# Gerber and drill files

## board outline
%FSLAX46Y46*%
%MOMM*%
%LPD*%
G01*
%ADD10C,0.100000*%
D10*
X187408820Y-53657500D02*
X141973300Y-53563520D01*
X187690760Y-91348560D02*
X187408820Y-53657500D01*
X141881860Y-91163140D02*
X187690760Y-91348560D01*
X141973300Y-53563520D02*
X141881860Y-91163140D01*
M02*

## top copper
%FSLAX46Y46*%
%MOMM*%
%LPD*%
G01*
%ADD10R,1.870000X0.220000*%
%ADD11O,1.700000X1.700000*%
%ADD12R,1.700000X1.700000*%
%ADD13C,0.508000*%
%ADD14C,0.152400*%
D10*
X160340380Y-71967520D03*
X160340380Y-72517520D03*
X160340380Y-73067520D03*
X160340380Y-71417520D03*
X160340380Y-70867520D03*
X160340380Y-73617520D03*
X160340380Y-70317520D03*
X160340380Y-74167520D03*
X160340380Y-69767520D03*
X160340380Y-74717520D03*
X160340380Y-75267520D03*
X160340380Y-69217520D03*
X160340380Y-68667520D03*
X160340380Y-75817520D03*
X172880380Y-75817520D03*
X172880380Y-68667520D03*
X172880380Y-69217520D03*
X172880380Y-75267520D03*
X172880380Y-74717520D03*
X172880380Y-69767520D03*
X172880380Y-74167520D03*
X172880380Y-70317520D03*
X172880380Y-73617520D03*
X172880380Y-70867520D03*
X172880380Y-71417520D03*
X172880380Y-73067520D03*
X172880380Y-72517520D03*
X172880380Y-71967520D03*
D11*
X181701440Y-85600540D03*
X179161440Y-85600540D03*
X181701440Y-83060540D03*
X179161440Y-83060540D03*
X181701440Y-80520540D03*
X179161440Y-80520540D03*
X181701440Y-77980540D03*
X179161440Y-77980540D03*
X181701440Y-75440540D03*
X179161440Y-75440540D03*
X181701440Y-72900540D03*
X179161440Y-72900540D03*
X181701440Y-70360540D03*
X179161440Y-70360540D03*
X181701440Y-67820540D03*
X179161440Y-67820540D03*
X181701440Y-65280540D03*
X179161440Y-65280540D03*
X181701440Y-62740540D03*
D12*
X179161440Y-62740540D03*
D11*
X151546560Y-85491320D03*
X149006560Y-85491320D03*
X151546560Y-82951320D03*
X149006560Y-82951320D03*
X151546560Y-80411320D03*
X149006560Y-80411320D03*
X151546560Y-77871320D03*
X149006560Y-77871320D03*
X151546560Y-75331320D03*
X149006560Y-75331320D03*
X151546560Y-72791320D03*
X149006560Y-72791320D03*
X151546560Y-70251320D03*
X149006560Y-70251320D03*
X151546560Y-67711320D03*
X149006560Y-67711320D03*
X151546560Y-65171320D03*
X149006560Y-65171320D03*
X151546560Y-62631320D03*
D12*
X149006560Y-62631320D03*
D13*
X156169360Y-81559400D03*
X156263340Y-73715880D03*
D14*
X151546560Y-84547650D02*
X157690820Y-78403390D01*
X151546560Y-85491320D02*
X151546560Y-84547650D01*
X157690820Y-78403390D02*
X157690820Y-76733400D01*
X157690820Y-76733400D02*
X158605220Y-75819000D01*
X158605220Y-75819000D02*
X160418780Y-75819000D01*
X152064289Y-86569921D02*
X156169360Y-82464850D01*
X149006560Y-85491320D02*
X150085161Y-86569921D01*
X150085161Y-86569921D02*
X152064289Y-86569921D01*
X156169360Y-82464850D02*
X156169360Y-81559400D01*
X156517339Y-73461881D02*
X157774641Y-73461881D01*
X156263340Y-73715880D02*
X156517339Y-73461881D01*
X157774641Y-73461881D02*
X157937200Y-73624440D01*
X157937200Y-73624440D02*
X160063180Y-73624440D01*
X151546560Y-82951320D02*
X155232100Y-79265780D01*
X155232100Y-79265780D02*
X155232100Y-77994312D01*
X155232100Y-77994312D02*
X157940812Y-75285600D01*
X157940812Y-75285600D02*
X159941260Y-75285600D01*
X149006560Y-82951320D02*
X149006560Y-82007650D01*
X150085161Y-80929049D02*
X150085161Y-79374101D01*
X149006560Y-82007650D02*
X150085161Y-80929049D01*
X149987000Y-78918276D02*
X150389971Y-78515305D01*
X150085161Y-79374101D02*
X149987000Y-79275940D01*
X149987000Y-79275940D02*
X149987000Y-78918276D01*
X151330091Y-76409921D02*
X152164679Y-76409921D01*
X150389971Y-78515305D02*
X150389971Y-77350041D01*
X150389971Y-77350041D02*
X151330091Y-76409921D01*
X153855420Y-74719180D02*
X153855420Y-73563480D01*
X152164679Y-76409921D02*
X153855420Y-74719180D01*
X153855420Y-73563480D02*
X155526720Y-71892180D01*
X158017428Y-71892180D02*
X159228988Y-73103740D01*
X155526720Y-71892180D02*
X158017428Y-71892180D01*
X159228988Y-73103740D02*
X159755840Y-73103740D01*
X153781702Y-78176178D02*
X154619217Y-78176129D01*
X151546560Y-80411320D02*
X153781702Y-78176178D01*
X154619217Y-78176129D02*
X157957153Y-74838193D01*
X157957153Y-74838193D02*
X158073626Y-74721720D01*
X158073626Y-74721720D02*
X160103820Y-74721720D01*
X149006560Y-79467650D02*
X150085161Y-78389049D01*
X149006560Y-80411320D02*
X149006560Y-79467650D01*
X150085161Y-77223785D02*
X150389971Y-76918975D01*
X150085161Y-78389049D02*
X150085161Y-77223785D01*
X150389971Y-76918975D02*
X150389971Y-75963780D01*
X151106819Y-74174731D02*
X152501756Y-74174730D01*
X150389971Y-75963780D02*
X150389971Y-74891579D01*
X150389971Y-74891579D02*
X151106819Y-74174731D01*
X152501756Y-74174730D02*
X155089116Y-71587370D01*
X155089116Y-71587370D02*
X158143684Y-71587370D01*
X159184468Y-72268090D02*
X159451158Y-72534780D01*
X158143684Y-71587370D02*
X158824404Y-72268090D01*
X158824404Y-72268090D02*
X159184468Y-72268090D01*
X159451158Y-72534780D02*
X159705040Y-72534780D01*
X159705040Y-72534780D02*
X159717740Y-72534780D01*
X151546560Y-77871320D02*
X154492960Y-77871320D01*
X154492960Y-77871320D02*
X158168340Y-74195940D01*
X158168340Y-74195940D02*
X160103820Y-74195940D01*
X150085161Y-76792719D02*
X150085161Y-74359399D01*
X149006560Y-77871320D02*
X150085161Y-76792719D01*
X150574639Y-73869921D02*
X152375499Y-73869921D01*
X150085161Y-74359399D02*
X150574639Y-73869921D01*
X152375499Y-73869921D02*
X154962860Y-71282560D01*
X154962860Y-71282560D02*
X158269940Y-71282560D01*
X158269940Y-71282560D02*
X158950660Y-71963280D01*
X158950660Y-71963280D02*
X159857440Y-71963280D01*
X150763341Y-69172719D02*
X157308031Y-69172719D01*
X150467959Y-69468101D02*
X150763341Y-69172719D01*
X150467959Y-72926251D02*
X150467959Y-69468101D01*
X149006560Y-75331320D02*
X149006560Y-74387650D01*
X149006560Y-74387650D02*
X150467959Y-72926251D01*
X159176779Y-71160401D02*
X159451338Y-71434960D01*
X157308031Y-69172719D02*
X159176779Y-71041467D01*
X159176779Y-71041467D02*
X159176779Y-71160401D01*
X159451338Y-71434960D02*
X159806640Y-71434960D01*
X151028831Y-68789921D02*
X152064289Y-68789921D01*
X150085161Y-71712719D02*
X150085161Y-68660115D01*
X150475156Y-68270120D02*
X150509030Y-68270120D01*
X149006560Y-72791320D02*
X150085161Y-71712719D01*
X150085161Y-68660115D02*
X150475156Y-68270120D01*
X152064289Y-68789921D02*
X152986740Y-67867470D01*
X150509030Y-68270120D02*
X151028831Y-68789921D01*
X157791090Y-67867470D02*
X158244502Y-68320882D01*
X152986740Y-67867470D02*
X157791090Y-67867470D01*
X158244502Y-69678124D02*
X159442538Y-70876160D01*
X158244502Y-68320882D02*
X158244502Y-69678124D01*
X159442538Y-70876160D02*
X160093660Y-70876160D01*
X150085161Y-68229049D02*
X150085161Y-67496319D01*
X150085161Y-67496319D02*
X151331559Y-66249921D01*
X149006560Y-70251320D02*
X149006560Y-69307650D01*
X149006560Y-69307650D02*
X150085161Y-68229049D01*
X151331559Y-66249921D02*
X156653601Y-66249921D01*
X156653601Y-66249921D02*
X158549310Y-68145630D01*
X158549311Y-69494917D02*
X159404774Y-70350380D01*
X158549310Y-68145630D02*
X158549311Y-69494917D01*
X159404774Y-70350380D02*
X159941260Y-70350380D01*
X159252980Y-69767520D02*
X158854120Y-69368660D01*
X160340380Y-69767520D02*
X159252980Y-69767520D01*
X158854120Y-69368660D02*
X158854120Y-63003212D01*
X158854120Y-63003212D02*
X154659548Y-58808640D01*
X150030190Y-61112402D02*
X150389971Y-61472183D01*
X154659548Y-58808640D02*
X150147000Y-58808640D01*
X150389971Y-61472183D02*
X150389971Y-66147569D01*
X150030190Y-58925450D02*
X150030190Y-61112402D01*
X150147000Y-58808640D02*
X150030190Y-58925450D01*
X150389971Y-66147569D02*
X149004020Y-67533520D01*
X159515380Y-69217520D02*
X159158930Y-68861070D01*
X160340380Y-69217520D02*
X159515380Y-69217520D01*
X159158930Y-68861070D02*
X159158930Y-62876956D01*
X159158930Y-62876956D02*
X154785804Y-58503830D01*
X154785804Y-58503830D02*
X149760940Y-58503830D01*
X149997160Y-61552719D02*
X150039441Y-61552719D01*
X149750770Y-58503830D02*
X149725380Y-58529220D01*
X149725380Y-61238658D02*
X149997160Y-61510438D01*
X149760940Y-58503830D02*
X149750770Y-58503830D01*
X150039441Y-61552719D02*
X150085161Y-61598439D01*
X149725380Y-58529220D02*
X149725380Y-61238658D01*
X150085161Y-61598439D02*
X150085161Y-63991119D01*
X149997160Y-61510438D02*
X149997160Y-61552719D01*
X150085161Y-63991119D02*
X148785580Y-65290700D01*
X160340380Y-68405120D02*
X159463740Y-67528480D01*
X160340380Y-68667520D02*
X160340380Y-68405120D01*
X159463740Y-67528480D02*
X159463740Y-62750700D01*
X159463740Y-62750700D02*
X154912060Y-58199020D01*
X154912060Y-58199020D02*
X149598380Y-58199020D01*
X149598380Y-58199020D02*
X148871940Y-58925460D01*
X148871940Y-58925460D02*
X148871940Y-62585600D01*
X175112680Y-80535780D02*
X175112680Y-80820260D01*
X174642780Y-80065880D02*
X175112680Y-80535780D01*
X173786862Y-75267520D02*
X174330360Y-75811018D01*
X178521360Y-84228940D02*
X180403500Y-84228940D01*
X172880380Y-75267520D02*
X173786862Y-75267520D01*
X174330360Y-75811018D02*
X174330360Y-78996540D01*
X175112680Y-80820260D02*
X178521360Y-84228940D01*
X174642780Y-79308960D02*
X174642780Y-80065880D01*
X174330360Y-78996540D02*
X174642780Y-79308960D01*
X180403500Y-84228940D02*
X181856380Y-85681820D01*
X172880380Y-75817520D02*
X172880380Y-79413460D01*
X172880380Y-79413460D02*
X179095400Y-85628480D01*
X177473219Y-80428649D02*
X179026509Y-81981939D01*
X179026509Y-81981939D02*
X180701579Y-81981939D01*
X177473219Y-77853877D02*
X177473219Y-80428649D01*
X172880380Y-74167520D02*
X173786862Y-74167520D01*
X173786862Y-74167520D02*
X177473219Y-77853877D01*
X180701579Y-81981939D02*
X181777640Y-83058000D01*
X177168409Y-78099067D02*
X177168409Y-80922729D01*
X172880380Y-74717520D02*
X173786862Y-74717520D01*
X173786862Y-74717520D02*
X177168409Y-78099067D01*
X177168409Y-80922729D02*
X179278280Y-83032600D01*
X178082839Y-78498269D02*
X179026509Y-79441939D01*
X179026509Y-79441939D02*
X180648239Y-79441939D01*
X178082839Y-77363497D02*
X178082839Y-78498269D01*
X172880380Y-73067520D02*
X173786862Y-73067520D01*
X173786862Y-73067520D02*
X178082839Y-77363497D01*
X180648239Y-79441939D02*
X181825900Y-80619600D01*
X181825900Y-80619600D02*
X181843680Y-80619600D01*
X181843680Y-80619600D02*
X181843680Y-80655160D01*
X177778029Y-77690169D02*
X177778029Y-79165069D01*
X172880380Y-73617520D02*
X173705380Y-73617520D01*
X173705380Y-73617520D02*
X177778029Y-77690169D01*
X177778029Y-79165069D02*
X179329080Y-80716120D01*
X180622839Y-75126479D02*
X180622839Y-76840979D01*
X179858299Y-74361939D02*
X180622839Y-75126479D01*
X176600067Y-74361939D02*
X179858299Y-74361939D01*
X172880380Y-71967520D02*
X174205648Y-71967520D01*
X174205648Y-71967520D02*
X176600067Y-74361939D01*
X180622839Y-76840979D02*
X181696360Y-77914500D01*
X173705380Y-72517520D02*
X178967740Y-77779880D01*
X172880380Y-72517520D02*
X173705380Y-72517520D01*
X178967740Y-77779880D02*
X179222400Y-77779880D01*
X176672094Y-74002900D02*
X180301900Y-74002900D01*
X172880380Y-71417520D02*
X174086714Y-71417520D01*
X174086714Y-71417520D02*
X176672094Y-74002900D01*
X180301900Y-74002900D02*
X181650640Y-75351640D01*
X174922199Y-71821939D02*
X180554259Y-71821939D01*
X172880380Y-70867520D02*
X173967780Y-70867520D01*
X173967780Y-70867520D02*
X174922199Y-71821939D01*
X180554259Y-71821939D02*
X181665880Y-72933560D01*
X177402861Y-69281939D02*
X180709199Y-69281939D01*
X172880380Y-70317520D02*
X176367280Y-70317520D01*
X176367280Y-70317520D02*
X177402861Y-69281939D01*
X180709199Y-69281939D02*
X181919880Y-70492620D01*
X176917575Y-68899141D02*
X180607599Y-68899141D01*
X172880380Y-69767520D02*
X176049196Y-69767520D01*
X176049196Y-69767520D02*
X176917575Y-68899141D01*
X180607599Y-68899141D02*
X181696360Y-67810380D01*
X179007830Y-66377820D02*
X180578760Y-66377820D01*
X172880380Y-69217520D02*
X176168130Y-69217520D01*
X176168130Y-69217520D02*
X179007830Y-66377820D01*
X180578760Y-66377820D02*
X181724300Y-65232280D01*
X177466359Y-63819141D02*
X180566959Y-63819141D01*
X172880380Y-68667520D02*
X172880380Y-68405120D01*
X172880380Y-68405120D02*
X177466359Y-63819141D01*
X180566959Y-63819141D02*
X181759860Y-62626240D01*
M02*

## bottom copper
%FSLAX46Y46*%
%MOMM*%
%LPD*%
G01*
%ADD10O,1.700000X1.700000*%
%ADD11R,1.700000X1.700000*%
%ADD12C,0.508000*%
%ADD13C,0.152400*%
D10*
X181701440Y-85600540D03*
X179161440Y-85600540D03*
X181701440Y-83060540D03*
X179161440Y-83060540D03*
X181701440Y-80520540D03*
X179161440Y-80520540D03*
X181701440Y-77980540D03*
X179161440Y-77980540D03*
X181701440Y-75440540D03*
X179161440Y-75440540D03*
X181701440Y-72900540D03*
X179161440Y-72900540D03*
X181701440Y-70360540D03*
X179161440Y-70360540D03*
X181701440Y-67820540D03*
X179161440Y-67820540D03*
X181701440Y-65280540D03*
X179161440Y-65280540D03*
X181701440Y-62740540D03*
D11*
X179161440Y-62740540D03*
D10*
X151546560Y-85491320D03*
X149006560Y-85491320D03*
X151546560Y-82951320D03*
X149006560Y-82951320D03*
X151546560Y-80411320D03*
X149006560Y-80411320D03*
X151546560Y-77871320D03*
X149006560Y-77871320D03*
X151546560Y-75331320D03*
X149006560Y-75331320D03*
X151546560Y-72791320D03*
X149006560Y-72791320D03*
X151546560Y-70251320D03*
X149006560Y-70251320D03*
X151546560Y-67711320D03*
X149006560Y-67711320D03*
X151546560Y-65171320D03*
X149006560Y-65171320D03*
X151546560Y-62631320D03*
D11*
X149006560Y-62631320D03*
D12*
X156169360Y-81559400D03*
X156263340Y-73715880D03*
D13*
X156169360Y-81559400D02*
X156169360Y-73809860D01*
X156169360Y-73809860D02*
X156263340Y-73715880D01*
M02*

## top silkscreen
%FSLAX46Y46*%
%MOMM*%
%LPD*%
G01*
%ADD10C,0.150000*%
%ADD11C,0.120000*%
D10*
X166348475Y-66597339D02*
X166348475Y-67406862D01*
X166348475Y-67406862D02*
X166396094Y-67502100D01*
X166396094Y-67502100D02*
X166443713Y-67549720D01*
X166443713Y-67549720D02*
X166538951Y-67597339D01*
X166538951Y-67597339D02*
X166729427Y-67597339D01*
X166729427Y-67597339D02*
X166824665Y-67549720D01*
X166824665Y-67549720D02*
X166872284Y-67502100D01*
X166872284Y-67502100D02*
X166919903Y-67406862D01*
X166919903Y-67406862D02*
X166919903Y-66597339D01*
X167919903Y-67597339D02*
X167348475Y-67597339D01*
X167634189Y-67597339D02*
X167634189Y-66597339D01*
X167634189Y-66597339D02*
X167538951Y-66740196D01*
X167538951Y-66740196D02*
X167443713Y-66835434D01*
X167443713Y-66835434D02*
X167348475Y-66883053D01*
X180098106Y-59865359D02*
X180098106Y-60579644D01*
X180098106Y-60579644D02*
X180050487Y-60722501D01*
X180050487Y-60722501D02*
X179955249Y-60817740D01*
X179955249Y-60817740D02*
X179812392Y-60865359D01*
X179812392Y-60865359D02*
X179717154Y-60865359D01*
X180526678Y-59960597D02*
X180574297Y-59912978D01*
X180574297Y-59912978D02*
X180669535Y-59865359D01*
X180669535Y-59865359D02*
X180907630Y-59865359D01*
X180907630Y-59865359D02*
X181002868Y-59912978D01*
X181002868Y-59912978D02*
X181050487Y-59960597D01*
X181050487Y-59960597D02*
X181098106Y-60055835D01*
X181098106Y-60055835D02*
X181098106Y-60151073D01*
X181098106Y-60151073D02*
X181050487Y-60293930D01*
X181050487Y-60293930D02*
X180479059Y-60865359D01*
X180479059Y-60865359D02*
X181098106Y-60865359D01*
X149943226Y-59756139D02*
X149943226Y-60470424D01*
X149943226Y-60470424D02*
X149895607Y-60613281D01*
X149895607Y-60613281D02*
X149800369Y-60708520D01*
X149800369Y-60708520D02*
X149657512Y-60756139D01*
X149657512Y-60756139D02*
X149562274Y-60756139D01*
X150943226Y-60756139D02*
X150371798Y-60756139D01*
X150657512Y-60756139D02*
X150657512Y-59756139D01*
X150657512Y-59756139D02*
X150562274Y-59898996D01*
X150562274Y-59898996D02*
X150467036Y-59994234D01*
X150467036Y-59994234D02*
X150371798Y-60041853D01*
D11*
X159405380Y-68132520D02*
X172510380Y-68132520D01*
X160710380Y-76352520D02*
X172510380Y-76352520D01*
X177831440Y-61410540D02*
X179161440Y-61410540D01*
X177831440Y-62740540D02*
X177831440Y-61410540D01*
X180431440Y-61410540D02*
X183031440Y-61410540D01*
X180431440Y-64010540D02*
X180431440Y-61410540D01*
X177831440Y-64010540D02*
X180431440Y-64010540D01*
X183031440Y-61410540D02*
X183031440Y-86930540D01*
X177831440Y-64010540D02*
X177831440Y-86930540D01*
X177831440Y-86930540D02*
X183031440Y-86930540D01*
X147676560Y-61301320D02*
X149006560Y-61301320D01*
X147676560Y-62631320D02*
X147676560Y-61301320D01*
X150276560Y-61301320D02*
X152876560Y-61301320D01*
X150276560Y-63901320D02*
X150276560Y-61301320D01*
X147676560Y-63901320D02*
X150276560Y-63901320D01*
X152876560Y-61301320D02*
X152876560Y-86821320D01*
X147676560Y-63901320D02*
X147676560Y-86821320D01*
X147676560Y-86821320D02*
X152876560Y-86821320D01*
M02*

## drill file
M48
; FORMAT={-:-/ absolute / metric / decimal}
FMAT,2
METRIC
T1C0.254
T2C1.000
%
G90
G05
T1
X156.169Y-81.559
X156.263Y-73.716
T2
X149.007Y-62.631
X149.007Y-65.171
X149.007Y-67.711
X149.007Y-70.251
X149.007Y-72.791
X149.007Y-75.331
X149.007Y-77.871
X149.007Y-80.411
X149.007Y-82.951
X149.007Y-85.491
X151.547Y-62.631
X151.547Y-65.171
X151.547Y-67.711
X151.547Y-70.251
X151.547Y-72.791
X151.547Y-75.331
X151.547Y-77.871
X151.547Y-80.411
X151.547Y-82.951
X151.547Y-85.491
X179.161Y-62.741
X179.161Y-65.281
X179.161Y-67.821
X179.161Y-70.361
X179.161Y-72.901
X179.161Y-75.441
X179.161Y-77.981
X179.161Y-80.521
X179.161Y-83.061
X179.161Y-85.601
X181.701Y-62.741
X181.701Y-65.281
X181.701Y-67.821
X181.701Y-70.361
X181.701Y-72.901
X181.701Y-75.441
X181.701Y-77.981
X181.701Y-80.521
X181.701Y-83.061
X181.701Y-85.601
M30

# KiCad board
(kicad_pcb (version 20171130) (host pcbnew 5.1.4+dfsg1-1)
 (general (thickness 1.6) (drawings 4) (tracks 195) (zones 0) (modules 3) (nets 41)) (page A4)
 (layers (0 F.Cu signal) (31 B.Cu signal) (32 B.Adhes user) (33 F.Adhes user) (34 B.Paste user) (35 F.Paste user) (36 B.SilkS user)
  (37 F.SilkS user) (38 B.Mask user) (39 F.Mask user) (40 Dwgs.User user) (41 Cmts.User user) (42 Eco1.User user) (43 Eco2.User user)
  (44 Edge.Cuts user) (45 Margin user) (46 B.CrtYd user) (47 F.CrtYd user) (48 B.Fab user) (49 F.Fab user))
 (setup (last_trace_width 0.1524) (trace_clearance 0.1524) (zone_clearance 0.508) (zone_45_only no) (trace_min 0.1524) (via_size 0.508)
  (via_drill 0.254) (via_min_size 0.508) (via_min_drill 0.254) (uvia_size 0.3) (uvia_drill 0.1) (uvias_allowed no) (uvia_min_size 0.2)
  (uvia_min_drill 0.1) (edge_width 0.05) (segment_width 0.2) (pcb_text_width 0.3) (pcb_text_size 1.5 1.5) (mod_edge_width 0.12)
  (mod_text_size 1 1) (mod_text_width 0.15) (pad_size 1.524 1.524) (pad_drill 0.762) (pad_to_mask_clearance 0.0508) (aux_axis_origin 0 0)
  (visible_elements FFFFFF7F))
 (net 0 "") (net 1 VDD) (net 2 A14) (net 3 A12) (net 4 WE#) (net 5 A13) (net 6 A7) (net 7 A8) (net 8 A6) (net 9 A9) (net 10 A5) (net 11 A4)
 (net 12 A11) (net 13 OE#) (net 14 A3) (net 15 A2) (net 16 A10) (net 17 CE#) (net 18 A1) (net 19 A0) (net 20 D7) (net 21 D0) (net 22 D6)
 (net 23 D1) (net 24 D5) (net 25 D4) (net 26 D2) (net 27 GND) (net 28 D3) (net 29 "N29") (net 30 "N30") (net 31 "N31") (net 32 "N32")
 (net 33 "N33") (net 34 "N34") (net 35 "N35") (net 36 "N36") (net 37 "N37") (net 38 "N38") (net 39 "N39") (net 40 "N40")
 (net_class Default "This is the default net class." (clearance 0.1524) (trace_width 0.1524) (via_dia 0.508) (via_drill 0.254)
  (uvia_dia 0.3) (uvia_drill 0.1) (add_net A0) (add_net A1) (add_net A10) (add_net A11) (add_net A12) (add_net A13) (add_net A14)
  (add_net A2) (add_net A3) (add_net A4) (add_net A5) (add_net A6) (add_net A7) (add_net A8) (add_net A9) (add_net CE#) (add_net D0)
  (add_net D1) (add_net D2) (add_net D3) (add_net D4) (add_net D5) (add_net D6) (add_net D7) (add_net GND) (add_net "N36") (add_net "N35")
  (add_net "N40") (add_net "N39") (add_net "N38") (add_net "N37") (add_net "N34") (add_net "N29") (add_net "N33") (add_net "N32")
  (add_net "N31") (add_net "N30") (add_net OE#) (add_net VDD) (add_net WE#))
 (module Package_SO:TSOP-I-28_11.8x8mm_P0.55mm (layer F.Cu) (at 166.61038 72.24252)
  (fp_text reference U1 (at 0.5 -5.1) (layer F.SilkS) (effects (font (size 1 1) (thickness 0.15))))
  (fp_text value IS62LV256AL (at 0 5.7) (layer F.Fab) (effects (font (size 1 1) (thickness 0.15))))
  (fp_line (start -7.205 -4.11) (end 5.9 -4.11) (layer F.SilkS) (width 0.12))
  (fp_line (start -5.9 4.11) (end 5.9 4.11) (layer F.SilkS) (width 0.12))
  (pad 7 smd rect (at -6.27 -0.275) (size 1.87 0.22) (layers F.Cu F.Paste F.Mask) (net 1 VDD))
  (pad 8 smd rect (at -6.27 0.275) (size 1.87 0.22) (layers F.Cu F.Paste F.Mask) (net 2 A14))
  (pad 9 smd rect (at -6.27 0.825) (size 1.87 0.22) (layers F.Cu F.Paste F.Mask) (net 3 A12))
  (pad 6 smd rect (at -6.27 -0.825) (size 1.87 0.22) (layers F.Cu F.Paste F.Mask) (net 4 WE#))
  (pad 5 smd rect (at -6.27 -1.375) (size 1.87 0.22) (layers F.Cu F.Paste F.Mask) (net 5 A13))
  (pad 10 smd rect (at -6.27 1.375) (size 1.87 0.22) (layers F.Cu F.Paste F.Mask) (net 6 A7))
  (pad 4 smd rect (at -6.27 -1.925) (size 1.87 0.22) (layers F.Cu F.Paste F.Mask) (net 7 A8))
  (pad 11 smd rect (at -6.27 1.925) (size 1.87 0.22) (layers F.Cu F.Paste F.Mask) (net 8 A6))
  (pad 3 smd rect (at -6.27 -2.475) (size 1.87 0.22) (layers F.Cu F.Paste F.Mask) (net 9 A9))
  (pad 12 smd rect (at -6.27 2.475) (size 1.87 0.22) (layers F.Cu F.Paste F.Mask) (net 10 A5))
  (pad 13 smd rect (at -6.27 3.025) (size 1.87 0.22) (layers F.Cu F.Paste F.Mask) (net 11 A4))
  (pad 2 smd rect (at -6.27 -3.025) (size 1.87 0.22) (layers F.Cu F.Paste F.Mask) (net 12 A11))
  (pad 1 smd rect (at -6.27 -3.575) (size 1.87 0.22) (layers F.Cu F.Paste F.Mask) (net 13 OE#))
  (pad 14 smd rect (at -6.27 3.575) (size 1.87 0.22) (layers F.Cu F.Paste F.Mask) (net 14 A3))
  (pad 15 smd rect (at 6.27 3.575) (size 1.87 0.22) (layers F.Cu F.Paste F.Mask) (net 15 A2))
  (pad 28 smd rect (at 6.27 -3.575) (size 1.87 0.22) (layers F.Cu F.Paste F.Mask) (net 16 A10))
  (pad 27 smd rect (at 6.27 -3.025) (size 1.87 0.22) (layers F.Cu F.Paste F.Mask) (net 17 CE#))
  (pad 16 smd rect (at 6.27 3.025) (size 1.87 0.22) (layers F.Cu F.Paste F.Mask) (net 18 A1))
  (pad 17 smd rect (at 6.27 2.475) (size 1.87 0.22) (layers F.Cu F.Paste F.Mask) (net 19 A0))
  (pad 26 smd rect (at 6.27 -2.475) (size 1.87 0.22) (layers F.Cu F.Paste F.Mask) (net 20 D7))
  (pad 18 smd rect (at 6.27 1.925) (size 1.87 0.22) (layers F.Cu F.Paste F.Mask) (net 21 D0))
  (pad 25 smd rect (at 6.27 -1.925) (size 1.87 0.22) (layers F.Cu F.Paste F.Mask) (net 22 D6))
  (pad 19 smd rect (at 6.27 1.375) (size 1.87 0.22) (layers F.Cu F.Paste F.Mask) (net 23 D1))
  (pad 24 smd rect (at 6.27 -1.375) (size 1.87 0.22) (layers F.Cu F.Paste F.Mask) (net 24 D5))
  (pad 23 smd rect (at 6.27 -0.825) (size 1.87 0.22) (layers F.Cu F.Paste F.Mask) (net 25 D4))
  (pad 20 smd rect (at 6.27 0.825) (size 1.87 0.22) (layers F.Cu F.Paste F.Mask) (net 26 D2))
  (pad 21 smd rect (at 6.27 0.275) (size 1.87 0.22) (layers F.Cu F.Paste F.Mask) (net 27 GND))
  (pad 22 smd rect (at 6.27 -0.275) (size 1.87 0.22) (layers F.Cu F.Paste F.Mask) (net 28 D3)))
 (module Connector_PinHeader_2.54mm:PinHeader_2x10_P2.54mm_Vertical (layer F.Cu) (at 179.16144 62.74054)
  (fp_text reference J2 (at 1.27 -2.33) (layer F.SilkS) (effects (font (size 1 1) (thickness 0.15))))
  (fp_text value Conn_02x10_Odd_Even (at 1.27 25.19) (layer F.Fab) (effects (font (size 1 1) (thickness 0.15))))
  (fp_line (start -1.33 -1.33) (end 0 -1.33) (layer F.SilkS) (width 0.12))
  (fp_line (start -1.33 0) (end -1.33 -1.33) (layer F.SilkS) (width 0.12))
  (fp_line (start 1.27 -1.33) (end 3.87 -1.33) (layer F.SilkS) (width 0.12))
  (fp_line (start 1.27 1.27) (end 1.27 -1.33) (layer F.SilkS) (width 0.12))
  (fp_line (start -1.33 1.27) (end 1.27 1.27) (layer F.SilkS) (width 0.12))
  (fp_line (start 3.87 -1.33) (end 3.87 24.19) (layer F.SilkS) (width 0.12))
  (fp_line (start -1.33 1.27) (end -1.33 24.19) (layer F.SilkS) (width 0.12))
  (fp_line (start -1.33 24.19) (end 3.87 24.19) (layer F.SilkS) (width 0.12))
  (pad 20 thru_hole oval (at 2.54 22.86) (size 1.7 1.7) (drill 1) (layers *.Cu *.Mask) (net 18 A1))
  (pad 19 thru_hole oval (at 0 22.86) (size 1.7 1.7) (drill 1) (layers *.Cu *.Mask) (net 15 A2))
  (pad 18 thru_hole oval (at 2.54 20.32) (size 1.7 1.7) (drill 1) (layers *.Cu *.Mask) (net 21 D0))
  (pad 17 thru_hole oval (at 0 20.32) (size 1.7 1.7) (drill 1) (layers *.Cu *.Mask) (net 19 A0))
  (pad 16 thru_hole oval (at 2.54 17.78) (size 1.7 1.7) (drill 1) (layers *.Cu *.Mask) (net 26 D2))
  (pad 15 thru_hole oval (at 0 17.78) (size 1.7 1.7) (drill 1) (layers *.Cu *.Mask) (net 23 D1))
  (pad 14 thru_hole oval (at 2.54 15.24) (size 1.7 1.7) (drill 1) (layers *.Cu *.Mask) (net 28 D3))
  (pad 13 thru_hole oval (at 0 15.24) (size 1.7 1.7) (drill 1) (layers *.Cu *.Mask) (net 27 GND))
  (pad 12 thru_hole oval (at 2.54 12.7) (size 1.7 1.7) (drill 1) (layers *.Cu *.Mask) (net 25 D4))
  (pad 11 thru_hole oval (at 0 12.7) (size 1.7 1.7) (drill 1) (layers *.Cu *.Mask) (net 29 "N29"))
  (pad 10 thru_hole oval (at 2.54 10.16) (size 1.7 1.7) (drill 1) (layers *.Cu *.Mask) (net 24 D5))
  (pad 9 thru_hole oval (at 0 10.16) (size 1.7 1.7) (drill 1) (layers *.Cu *.Mask) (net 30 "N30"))
  (pad 8 thru_hole oval (at 2.54 7.62) (size 1.7 1.7) (drill 1) (layers *.Cu *.Mask) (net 22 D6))
  (pad 7 thru_hole oval (at 0 7.62) (size 1.7 1.7) (drill 1) (layers *.Cu *.Mask) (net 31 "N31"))
  (pad 6 thru_hole oval (at 2.54 5.08) (size 1.7 1.7) (drill 1) (layers *.Cu *.Mask) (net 20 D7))
  (pad 5 thru_hole oval (at 0 5.08) (size 1.7 1.7) (drill 1) (layers *.Cu *.Mask) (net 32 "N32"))
  (pad 4 thru_hole oval (at 2.54 2.54) (size 1.7 1.7) (drill 1) (layers *.Cu *.Mask) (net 17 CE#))
  (pad 3 thru_hole oval (at 0 2.54) (size 1.7 1.7) (drill 1) (layers *.Cu *.Mask) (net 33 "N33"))
  (pad 2 thru_hole oval (at 2.54 0) (size 1.7 1.7) (drill 1) (layers *.Cu *.Mask) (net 16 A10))
  (pad 1 thru_hole rect (at 0 0) (size 1.7 1.7) (drill 1) (layers *.Cu *.Mask) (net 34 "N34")))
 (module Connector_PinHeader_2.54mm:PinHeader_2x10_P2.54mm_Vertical (layer F.Cu) (at 149.00656 62.63132)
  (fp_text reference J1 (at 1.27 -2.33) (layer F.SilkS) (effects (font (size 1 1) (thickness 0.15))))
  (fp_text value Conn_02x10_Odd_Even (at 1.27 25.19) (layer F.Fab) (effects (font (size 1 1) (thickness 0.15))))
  (fp_line (start -1.33 -1.33) (end 0 -1.33) (layer F.SilkS) (width 0.12))
  (fp_line (start -1.33 0) (end -1.33 -1.33) (layer F.SilkS) (width 0.12))
  (fp_line (start 1.27 -1.33) (end 3.87 -1.33) (layer F.SilkS) (width 0.12))
  (fp_line (start 1.27 1.27) (end 1.27 -1.33) (layer F.SilkS) (width 0.12))
  (fp_line (start -1.33 1.27) (end 1.27 1.27) (layer F.SilkS) (width 0.12))
  (fp_line (start 3.87 -1.33) (end 3.87 24.19) (layer F.SilkS) (width 0.12))
  (fp_line (start -1.33 1.27) (end -1.33 24.19) (layer F.SilkS) (width 0.12))
  (fp_line (start -1.33 24.19) (end 3.87 24.19) (layer F.SilkS) (width 0.12))
  (pad 20 thru_hole oval (at 2.54 22.86) (size 1.7 1.7) (drill 1) (layers *.Cu *.Mask) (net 14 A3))
  (pad 19 thru_hole oval (at 0 22.86) (size 1.7 1.7) (drill 1) (layers *.Cu *.Mask) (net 6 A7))
  (pad 18 thru_hole oval (at 2.54 20.32) (size 1.7 1.7) (drill 1) (layers *.Cu *.Mask) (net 11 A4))
  (pad 17 thru_hole oval (at 0 20.32) (size 1.7 1.7) (drill 1) (layers *.Cu *.Mask) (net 3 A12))
  (pad 16 thru_hole oval (at 2.54 17.78) (size 1.7 1.7) (drill 1) (layers *.Cu *.Mask) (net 10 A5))
  (pad 15 thru_hole oval (at 0 17.78) (size 1.7 1.7) (drill 1) (layers *.Cu *.Mask) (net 2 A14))
  (pad 14 thru_hole oval (at 2.54 15.24) (size 1.7 1.7) (drill 1) (layers *.Cu *.Mask) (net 8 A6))
  (pad 13 thru_hole oval (at 0 15.24) (size 1.7 1.7) (drill 1) (layers *.Cu *.Mask) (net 1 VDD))
  (pad 12 thru_hole oval (at 2.54 12.7) (size 1.7 1.7) (drill 1) (layers *.Cu *.Mask) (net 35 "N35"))
  (pad 11 thru_hole oval (at 0 12.7) (size 1.7 1.7) (drill 1) (layers *.Cu *.Mask) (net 4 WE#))
  (pad 10 thru_hole oval (at 2.54 10.16) (size 1.7 1.7) (drill 1) (layers *.Cu *.Mask) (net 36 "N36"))
  (pad 9 thru_hole oval (at 0 10.16) (size 1.7 1.7) (drill 1) (layers *.Cu *.Mask) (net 5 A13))
  (pad 8 thru_hole oval (at 2.54 7.62) (size 1.7 1.7) (drill 1) (layers *.Cu *.Mask) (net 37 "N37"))
  (pad 7 thru_hole oval (at 0 7.62) (size 1.7 1.7) (drill 1) (layers *.Cu *.Mask) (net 7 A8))
  (pad 6 thru_hole oval (at 2.54 5.08) (size 1.7 1.7) (drill 1) (layers *.Cu *.Mask) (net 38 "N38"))
  (pad 5 thru_hole oval (at 0 5.08) (size 1.7 1.7) (drill 1) (layers *.Cu *.Mask) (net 9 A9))
  (pad 4 thru_hole oval (at 2.54 2.54) (size 1.7 1.7) (drill 1) (layers *.Cu *.Mask) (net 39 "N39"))
  (pad 3 thru_hole oval (at 0 2.54) (size 1.7 1.7) (drill 1) (layers *.Cu *.Mask) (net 12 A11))
  (pad 2 thru_hole oval (at 2.54 0) (size 1.7 1.7) (drill 1) (layers *.Cu *.Mask) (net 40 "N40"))
  (pad 1 thru_hole rect (at 0 0) (size 1.7 1.7) (drill 1) (layers *.Cu *.Mask) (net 13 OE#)))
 (gr_line (start 187.40882 53.6575) (end 141.9733 53.56352) (layer Edge.Cuts) (width 0.1))
 (gr_line (start 187.69076 91.34856) (end 187.40882 53.6575) (layer Edge.Cuts) (width 0.1))
 (gr_line (start 141.88186 91.16314) (end 187.69076 91.34856) (layer Edge.Cuts) (width 0.1))
 (gr_line (start 141.9733 53.56352) (end 141.88186 91.16314) (layer Edge.Cuts) (width 0.1))
 (segment (start 151.54656 84.54765) (end 157.69082 78.40339) (width 0.1524) (layer F.Cu) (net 14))
 (segment (start 151.54656 85.49132) (end 151.54656 84.54765) (width 0.1524) (layer F.Cu) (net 14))
 (segment (start 157.69082 78.40339) (end 157.69082 76.7334) (width 0.1524) (layer F.Cu) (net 14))
 (segment (start 157.69082 76.7334) (end 158.60522 75.819) (width 0.1524) (layer F.Cu) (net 14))
 (segment (start 158.60522 75.819) (end 160.41878 75.819) (width 0.1524) (layer F.Cu) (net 14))
 (segment (start 152.064289 86.569921) (end 156.16936 82.46485) (width 0.1524) (layer F.Cu) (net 6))
 (segment (start 149.00656 85.49132) (end 150.085161 86.569921) (width 0.1524) (layer F.Cu) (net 6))
 (segment (start 150.085161 86.569921) (end 152.064289 86.569921) (width 0.1524) (layer F.Cu) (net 6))
 (via (at 156.16936 81.5594) (size 0.508) (drill 0.254) (layers F.Cu B.Cu) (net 6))
 (segment (start 156.16936 82.46485) (end 156.16936 81.5594) (width 0.1524) (layer F.Cu) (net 6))
 (via (at 156.26334 73.71588) (size 0.508) (drill 0.254) (layers F.Cu B.Cu) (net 6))
 (segment (start 156.16936 81.5594) (end 156.16936 73.80986) (width 0.1524) (layer B.Cu) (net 6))
 (segment (start 156.16936 73.80986) (end 156.26334 73.71588) (width 0.1524) (layer B.Cu) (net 6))
 (segment (start 156.517339 73.461881) (end 157.774641 73.461881) (width 0.1524) (layer F.Cu) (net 6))
 (segment (start 156.26334 73.71588) (end 156.517339 73.461881) (width 0.1524) (layer F.Cu) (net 6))
 (segment (start 157.774641 73.461881) (end 157.9372 73.62444) (width 0.1524) (layer F.Cu) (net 6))
 (segment (start 157.9372 73.62444) (end 160.06318 73.62444) (width 0.1524) (layer F.Cu) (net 6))
 (segment (start 151.54656 82.95132) (end 155.2321 79.26578) (width 0.1524) (layer F.Cu) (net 11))
 (segment (start 155.2321 79.26578) (end 155.2321 77.994312) (width 0.1524) (layer F.Cu) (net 11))
 (segment (start 155.2321 77.994312) (end 157.940812 75.2856) (width 0.1524) (layer F.Cu) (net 11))
 (segment (start 157.940812 75.2856) (end 159.94126 75.2856) (width 0.1524) (layer F.Cu) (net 11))
 (segment (start 149.00656 82.95132) (end 149.00656 82.00765) (width 0.1524) (layer F.Cu) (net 3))
 (segment (start 150.085161 80.929049) (end 150.085161 79.374101) (width 0.1524) (layer F.Cu) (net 3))
 (segment (start 149.00656 82.00765) (end 150.085161 80.929049) (width 0.1524) (layer F.Cu) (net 3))
 (segment (start 149.987 78.918276) (end 150.389971 78.515305) (width 0.1524) (layer F.Cu) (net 3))
 (segment (start 150.085161 79.374101) (end 149.987 79.27594) (width 0.1524) (layer F.Cu) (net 3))
 (segment (start 149.987 79.27594) (end 149.987 78.918276) (width 0.1524) (layer F.Cu) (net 3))
 (segment (start 151.330091 76.409921) (end 152.164679 76.409921) (width 0.1524) (layer F.Cu) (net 3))
 (segment (start 150.389971 78.515305) (end 150.389971 77.350041) (width 0.1524) (layer F.Cu) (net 3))
 (segment (start 150.389971 77.350041) (end 151.330091 76.409921) (width 0.1524) (layer F.Cu) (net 3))
 (segment (start 153.85542 74.71918) (end 153.85542 73.56348) (width 0.1524) (layer F.Cu) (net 3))
 (segment (start 152.164679 76.409921) (end 153.85542 74.71918) (width 0.1524) (layer F.Cu) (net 3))
 (segment (start 153.85542 73.56348) (end 155.52672 71.89218) (width 0.1524) (layer F.Cu) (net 3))
 (segment (start 158.017428 71.89218) (end 159.228988 73.10374) (width 0.1524) (layer F.Cu) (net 3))
 (segment (start 155.52672 71.89218) (end 158.017428 71.89218) (width 0.1524) (layer F.Cu) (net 3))
 (segment (start 159.228988 73.10374) (end 159.75584 73.10374) (width 0.1524) (layer F.Cu) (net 3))
 (segment (start 153.781702 78.176178) (end 154.619217 78.176129) (width 0.1524) (layer F.Cu) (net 10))
 (segment (start 151.54656 80.41132) (end 153.781702 78.176178) (width 0.1524) (layer F.Cu) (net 10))
 (segment (start 154.619217 78.176129) (end 157.957153 74.838193) (width 0.1524) (layer F.Cu) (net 10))
 (segment (start 157.957153 74.838193) (end 158.073626 74.72172) (width 0.1524) (layer F.Cu) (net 10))
 (segment (start 158.073626 74.72172) (end 160.10382 74.72172) (width 0.1524) (layer F.Cu) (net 10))
 (segment (start 149.00656 79.46765) (end 150.085161 78.389049) (width 0.1524) (layer F.Cu) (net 2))
 (segment (start 149.00656 80.41132) (end 149.00656 79.46765) (width 0.1524) (layer F.Cu) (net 2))
 (segment (start 150.085161 77.223785) (end 150.389971 76.918975) (width 0.1524) (layer F.Cu) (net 2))
 (segment (start 150.085161 78.389049) (end 150.085161 77.223785) (width 0.1524) (layer F.Cu) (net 2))
 (segment (start 150.389971 76.918975) (end 150.389971 75.96378) (width 0.1524) (layer F.Cu) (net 2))
 (segment (start 151.106819 74.174731) (end 152.501756 74.17473) (width 0.1524) (layer F.Cu) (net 2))
 (segment (start 150.389971 75.96378) (end 150.389971 74.891579) (width 0.1524) (layer F.Cu) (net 2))
 (segment (start 150.389971 74.891579) (end 151.106819 74.174731) (width 0.1524) (layer F.Cu) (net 2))
 (segment (start 152.501756 74.17473) (end 155.089116 71.58737) (width 0.1524) (layer F.Cu) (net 2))
 (segment (start 155.089116 71.58737) (end 158.143684 71.58737) (width 0.1524) (layer F.Cu) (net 2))
 (segment (start 159.184468 72.26809) (end 159.451158 72.53478) (width 0.1524) (layer F.Cu) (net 2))
 (segment (start 158.143684 71.58737) (end 158.824404 72.26809) (width 0.1524) (layer F.Cu) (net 2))
 (segment (start 158.824404 72.26809) (end 159.184468 72.26809) (width 0.1524) (layer F.Cu) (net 2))
 (segment (start 159.451158 72.53478) (end 159.70504 72.53478) (width 0.1524) (layer F.Cu) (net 2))
 (segment (start 159.70504 72.53478) (end 159.71774 72.53478) (width 0.1524) (layer F.Cu) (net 2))
 (segment (start 151.54656 77.87132) (end 154.49296 77.87132) (width 0.1524) (layer F.Cu) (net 8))
 (segment (start 154.49296 77.87132) (end 158.16834 74.19594) (width 0.1524) (layer F.Cu) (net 8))
 (segment (start 158.16834 74.19594) (end 160.10382 74.19594) (width 0.1524) (layer F.Cu) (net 8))
 (segment (start 150.085161 76.792719) (end 150.085161 74.359399) (width 0.1524) (layer F.Cu) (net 1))
 (segment (start 149.00656 77.87132) (end 150.085161 76.792719) (width 0.1524) (layer F.Cu) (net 1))
 (segment (start 150.574639 73.869921) (end 152.375499 73.869921) (width 0.1524) (layer F.Cu) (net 1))
 (segment (start 150.085161 74.359399) (end 150.574639 73.869921) (width 0.1524) (layer F.Cu) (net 1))
 (segment (start 152.375499 73.869921) (end 154.96286 71.28256) (width 0.1524) (layer F.Cu) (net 1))
 (segment (start 154.96286 71.28256) (end 158.26994 71.28256) (width 0.1524) (layer F.Cu) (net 1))
 (segment (start 158.26994 71.28256) (end 158.95066 71.96328) (width 0.1524) (layer F.Cu) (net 1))
 (segment (start 158.95066 71.96328) (end 159.85744 71.96328) (width 0.1524) (layer F.Cu) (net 1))
 (segment (start 150.763341 69.172719) (end 157.308031 69.172719) (width 0.1524) (layer F.Cu) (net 4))
 (segment (start 150.467959 69.468101) (end 150.763341 69.172719) (width 0.1524) (layer F.Cu) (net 4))
 (segment (start 150.467959 72.926251) (end 150.467959 69.468101) (width 0.1524) (layer F.Cu) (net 4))
 (segment (start 149.00656 75.33132) (end 149.00656 74.38765) (width 0.1524) (layer F.Cu) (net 4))
 (segment (start 149.00656 74.38765) (end 150.467959 72.926251) (width 0.1524) (layer F.Cu) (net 4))
 (segment (start 159.176779 71.160401) (end 159.451338 71.43496) (width 0.1524) (layer F.Cu) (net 4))
 (segment (start 157.308031 69.172719) (end 159.176779 71.041467) (width 0.1524) (layer F.Cu) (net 4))
 (segment (start 159.176779 71.041467) (end 159.176779 71.160401) (width 0.1524) (layer F.Cu) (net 4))
 (segment (start 159.451338 71.43496) (end 159.80664 71.43496) (width 0.1524) (layer F.Cu) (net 4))
 (segment (start 151.028831 68.789921) (end 152.064289 68.789921) (width 0.1524) (layer F.Cu) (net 5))
 (segment (start 150.085161 71.712719) (end 150.085161 68.660115) (width 0.1524) (layer F.Cu) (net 5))
 (segment (start 150.475156 68.27012) (end 150.50903 68.27012) (width 0.1524) (layer F.Cu) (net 5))
 (segment (start 149.00656 72.79132) (end 150.085161 71.712719) (width 0.1524) (layer F.Cu) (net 5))
 (segment (start 150.085161 68.660115) (end 150.475156 68.27012) (width 0.1524) (layer F.Cu) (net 5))
 (segment (start 152.064289 68.789921) (end 152.98674 67.86747) (width 0.1524) (layer F.Cu) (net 5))
 (segment (start 150.50903 68.27012) (end 151.028831 68.789921) (width 0.1524) (layer F.Cu) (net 5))
 (segment (start 157.79109 67.86747) (end 158.244502 68.320882) (width 0.1524) (layer F.Cu) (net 5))
 (segment (start 152.98674 67.86747) (end 157.79109 67.86747) (width 0.1524) (layer F.Cu) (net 5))
 (segment (start 158.244502 69.678124) (end 159.442538 70.87616) (width 0.1524) (layer F.Cu) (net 5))
 (segment (start 158.244502 68.320882) (end 158.244502 69.678124) (width 0.1524) (layer F.Cu) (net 5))
 (segment (start 159.442538 70.87616) (end 160.09366 70.87616) (width 0.1524) (layer F.Cu) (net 5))
 (segment (start 150.085161 68.229049) (end 150.085161 67.496319) (width 0.1524) (layer F.Cu) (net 7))
 (segment (start 150.085161 67.496319) (end 151.331559 66.249921) (width 0.1524) (layer F.Cu) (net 7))
 (segment (start 149.00656 70.25132) (end 149.00656 69.30765) (width 0.1524) (layer F.Cu) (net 7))
 (segment (start 149.00656 69.30765) (end 150.085161 68.229049) (width 0.1524) (layer F.Cu) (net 7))
 (segment (start 151.331559 66.249921) (end 156.653601 66.249921) (width 0.1524) (layer F.Cu) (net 7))
 (segment (start 156.653601 66.249921) (end 158.54931 68.14563) (width 0.1524) (layer F.Cu) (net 7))
 (segment (start 158.549311 69.494917) (end 159.404774 70.35038) (width 0.1524) (layer F.Cu) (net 7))
 (segment (start 158.54931 68.14563) (end 158.549311 69.494917) (width 0.1524) (layer F.Cu) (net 7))
 (segment (start 159.404774 70.35038) (end 159.94126 70.35038) (width 0.1524) (layer F.Cu) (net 7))
 (segment (start 159.25298 69.76752) (end 158.85412 69.36866) (width 0.1524) (layer F.Cu) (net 9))
 (segment (start 160.34038 69.76752) (end 159.25298 69.76752) (width 0.1524) (layer F.Cu) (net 9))
 (segment (start 158.85412 69.36866) (end 158.85412 63.003212) (width 0.1524) (layer F.Cu) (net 9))
 (segment (start 158.85412 63.003212) (end 154.659548 58.80864) (width 0.1524) (layer F.Cu) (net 9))
 (segment (start 150.03019 61.112402) (end 150.389971 61.472183) (width 0.1524) (layer F.Cu) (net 9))
 (segment (start 154.659548 58.80864) (end 150.147 58.80864) (width 0.1524) (layer F.Cu) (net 9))
 (segment (start 150.389971 61.472183) (end 150.389971 66.147569) (width 0.1524) (layer F.Cu) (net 9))
 (segment (start 150.03019 58.92545) (end 150.03019 61.112402) (width 0.1524) (layer F.Cu) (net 9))
 (segment (start 150.147 58.80864) (end 150.03019 58.92545) (width 0.1524) (layer F.Cu) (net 9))
 (segment (start 150.389971 66.147569) (end 149.00402 67.53352) (width 0.1524) (layer F.Cu) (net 9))
 (segment (start 159.51538 69.21752) (end 159.15893 68.86107) (width 0.1524) (layer F.Cu) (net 12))
 (segment (start 160.34038 69.21752) (end 159.51538 69.21752) (width 0.1524) (layer F.Cu) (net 12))
 (segment (start 159.15893 68.86107) (end 159.15893 62.876956) (width 0.1524) (layer F.Cu) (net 12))
 (segment (start 159.15893 62.876956) (end 154.785804 58.50383) (width 0.1524) (layer F.Cu) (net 12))
 (segment (start 154.785804 58.50383) (end 149.76094 58.50383) (width 0.1524) (layer F.Cu) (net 12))
 (segment (start 149.99716 61.552719) (end 150.039441 61.552719) (width 0.1524) (layer F.Cu) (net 12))
 (segment (start 149.75077 58.50383) (end 149.72538 58.52922) (width 0.1524) (layer F.Cu) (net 12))
 (segment (start 149.72538 61.238658) (end 149.99716 61.510438) (width 0.1524) (layer F.Cu) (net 12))
 (segment (start 149.76094 58.50383) (end 149.75077 58.50383) (width 0.1524) (layer F.Cu) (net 12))
 (segment (start 150.039441 61.552719) (end 150.085161 61.598439) (width 0.1524) (layer F.Cu) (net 12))
 (segment (start 149.72538 58.52922) (end 149.72538 61.238658) (width 0.1524) (layer F.Cu) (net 12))
 (segment (start 150.085161 61.598439) (end 150.085161 63.991119) (width 0.1524) (layer F.Cu) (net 12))
 (segment (start 149.99716 61.510438) (end 149.99716 61.552719) (width 0.1524) (layer F.Cu) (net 12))
 (segment (start 150.085161 63.991119) (end 148.78558 65.2907) (width 0.1524) (layer F.Cu) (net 12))
 (segment (start 160.34038 68.40512) (end 159.46374 67.52848) (width 0.1524) (layer F.Cu) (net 13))
 (segment (start 160.34038 68.66752) (end 160.34038 68.40512) (width 0.1524) (layer F.Cu) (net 13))
 (segment (start 159.46374 67.52848) (end 159.46374 62.7507) (width 0.1524) (layer F.Cu) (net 13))
 (segment (start 159.46374 62.7507) (end 154.91206 58.19902) (width 0.1524) (layer F.Cu) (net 13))
 (segment (start 154.91206 58.19902) (end 149.59838 58.19902) (width 0.1524) (layer F.Cu) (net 13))
 (segment (start 149.59838 58.19902) (end 148.87194 58.92546) (width 0.1524) (layer F.Cu) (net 13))
 (segment (start 148.87194 58.92546) (end 148.87194 62.5856) (width 0.1524) (layer F.Cu) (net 13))
 (segment (start 175.11268 80.53578) (end 175.11268 80.82026) (width 0.1524) (layer F.Cu) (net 18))
 (segment (start 174.64278 80.06588) (end 175.11268 80.53578) (width 0.1524) (layer F.Cu) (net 18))
 (segment (start 173.786862 75.26752) (end 174.33036 75.811018) (width 0.1524) (layer F.Cu) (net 18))
 (segment (start 178.52136 84.22894) (end 180.4035 84.22894) (width 0.1524) (layer F.Cu) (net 18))
 (segment (start 172.88038 75.26752) (end 173.786862 75.26752) (width 0.1524) (layer F.Cu) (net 18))
 (segment (start 174.33036 75.811018) (end 174.33036 78.99654) (width 0.1524) (layer F.Cu) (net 18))
 (segment (start 175.11268 80.82026) (end 178.52136 84.22894) (width 0.1524) (layer F.Cu) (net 18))
 (segment (start 174.64278 79.30896) (end 174.64278 80.06588) (width 0.1524) (layer F.Cu) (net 18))
 (segment (start 174.33036 78.99654) (end 174.64278 79.30896) (width 0.1524) (layer F.Cu) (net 18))
 (segment (start 180.4035 84.22894) (end 181.85638 85.68182) (width 0.1524) (layer F.Cu) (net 18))
 (segment (start 172.88038 75.81752) (end 172.88038 79.41346) (width 0.1524) (layer F.Cu) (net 15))
 (segment (start 172.88038 79.41346) (end 179.0954 85.62848) (width 0.1524) (layer F.Cu) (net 15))
 (segment (start 177.473219 80.428649) (end 179.026509 81.981939) (width 0.1524) (layer F.Cu) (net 21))
 (segment (start 179.026509 81.981939) (end 180.701579 81.981939) (width 0.1524) (layer F.Cu) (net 21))
 (segment (start 177.473219 77.853877) (end 177.473219 80.428649) (width 0.1524) (layer F.Cu) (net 21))
 (segment (start 172.88038 74.16752) (end 173.786862 74.16752) (width 0.1524) (layer F.Cu) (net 21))
 (segment (start 173.786862 74.16752) (end 177.473219 77.853877) (width 0.1524) (layer F.Cu) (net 21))
 (segment (start 180.701579 81.981939) (end 181.77764 83.058) (width 0.1524) (layer F.Cu) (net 21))
 (segment (start 177.168409 78.099067) (end 177.168409 80.922729) (width 0.1524) (layer F.Cu) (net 19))
 (segment (start 172.88038 74.71752) (end 173.786862 74.71752) (width 0.1524) (layer F.Cu) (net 19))
 (segment (start 173.786862 74.71752) (end 177.168409 78.099067) (width 0.1524) (layer F.Cu) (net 19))
 (segment (start 177.168409 80.922729) (end 179.27828 83.0326) (width 0.1524) (layer F.Cu) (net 19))
 (segment (start 178.082839 78.498269) (end 179.026509 79.441939) (width 0.1524) (layer F.Cu) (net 26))
 (segment (start 179.026509 79.441939) (end 180.648239 79.441939) (width 0.1524) (layer F.Cu) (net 26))
 (segment (start 178.082839 77.363497) (end 178.082839 78.498269) (width 0.1524) (layer F.Cu) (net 26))
 (segment (start 172.88038 73.06752) (end 173.786862 73.06752) (width 0.1524) (layer F.Cu) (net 26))
 (segment (start 173.786862 73.06752) (end 178.082839 77.363497) (width 0.1524) (layer F.Cu) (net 26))
 (segment (start 180.648239 79.441939) (end 181.8259 80.6196) (width 0.1524) (layer F.Cu) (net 26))
 (segment (start 181.8259 80.6196) (end 181.84368 80.6196) (width 0.1524) (layer F.Cu) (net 26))
 (segment (start 181.84368 80.6196) (end 181.84368 80.65516) (width 0.1524) (layer F.Cu) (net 26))
 (segment (start 177.778029 77.690169) (end 177.778029 79.165069) (width 0.1524) (layer F.Cu) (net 23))
 (segment (start 172.88038 73.61752) (end 173.70538 73.61752) (width 0.1524) (layer F.Cu) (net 23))
 (segment (start 173.70538 73.61752) (end 177.778029 77.690169) (width 0.1524) (layer F.Cu) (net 23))
 (segment (start 177.778029 79.165069) (end 179.32908 80.71612) (width 0.1524) (layer F.Cu) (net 23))
 (segment (start 180.622839 75.126479) (end 180.622839 76.840979) (width 0.1524) (layer F.Cu) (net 28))
 (segment (start 179.858299 74.361939) (end 180.622839 75.126479) (width 0.1524) (layer F.Cu) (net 28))
 (segment (start 176.600067 74.361939) (end 179.858299 74.361939) (width 0.1524) (layer F.Cu) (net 28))
 (segment (start 172.88038 71.96752) (end 174.205648 71.96752) (width 0.1524) (layer F.Cu) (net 28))
 (segment (start 174.205648 71.96752) (end 176.600067 74.361939) (width 0.1524) (layer F.Cu) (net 28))
 (segment (start 180.622839 76.840979) (end 181.69636 77.9145) (width 0.1524) (layer F.Cu) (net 28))
 (segment (start 173.70538 72.51752) (end 178.96774 77.77988) (width 0.1524) (layer F.Cu) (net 27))
 (segment (start 172.88038 72.51752) (end 173.70538 72.51752) (width 0.1524) (layer F.Cu) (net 27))
 (segment (start 178.96774 77.77988) (end 179.2224 77.77988) (width 0.1524) (layer F.Cu) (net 27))
 (segment (start 176.672094 74.0029) (end 180.3019 74.0029) (width 0.1524) (layer F.Cu) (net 25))
 (segment (start 172.88038 71.41752) (end 174.086714 71.41752) (width 0.1524) (layer F.Cu) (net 25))
 (segment (start 174.086714 71.41752) (end 176.672094 74.0029) (width 0.1524) (layer F.Cu) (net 25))
 (segment (start 180.3019 74.0029) (end 181.65064 75.35164) (width 0.1524) (layer F.Cu) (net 25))
 (segment (start 174.922199 71.821939) (end 180.554259 71.821939) (width 0.1524) (layer F.Cu) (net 24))
 (segment (start 172.88038 70.86752) (end 173.96778 70.86752) (width 0.1524) (layer F.Cu) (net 24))
 (segment (start 173.96778 70.86752) (end 174.922199 71.821939) (width 0.1524) (layer F.Cu) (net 24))
 (segment (start 180.554259 71.821939) (end 181.66588 72.93356) (width 0.1524) (layer F.Cu) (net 24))
 (segment (start 177.402861 69.281939) (end 180.709199 69.281939) (width 0.1524) (layer F.Cu) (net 22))
 (segment (start 172.88038 70.31752) (end 176.36728 70.31752) (width 0.1524) (layer F.Cu) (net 22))
 (segment (start 176.36728 70.31752) (end 177.402861 69.281939) (width 0.1524) (layer F.Cu) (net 22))
 (segment (start 180.709199 69.281939) (end 181.91988 70.49262) (width 0.1524) (layer F.Cu) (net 22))
 (segment (start 176.917575 68.899141) (end 180.607599 68.899141) (width 0.1524) (layer F.Cu) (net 20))
 (segment (start 172.88038 69.76752) (end 176.049196 69.76752) (width 0.1524) (layer F.Cu) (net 20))
 (segment (start 176.049196 69.76752) (end 176.917575 68.899141) (width 0.1524) (layer F.Cu) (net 20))
 (segment (start 180.607599 68.899141) (end 181.69636 67.81038) (width 0.1524) (layer F.Cu) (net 20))
 (segment (start 179.00783 66.37782) (end 180.57876 66.37782) (width 0.1524) (layer F.Cu) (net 17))
 (segment (start 172.88038 69.21752) (end 176.16813 69.21752) (width 0.1524) (layer F.Cu) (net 17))
 (segment (start 176.16813 69.21752) (end 179.00783 66.37782) (width 0.1524) (layer F.Cu) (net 17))
 (segment (start 180.57876 66.37782) (end 181.7243 65.23228) (width 0.1524) (layer F.Cu) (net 17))
 (segment (start 177.466359 63.819141) (end 180.566959 63.819141) (width 0.1524) (layer F.Cu) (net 16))
 (segment (start 172.88038 68.66752) (end 172.88038 68.40512) (width 0.1524) (layer F.Cu) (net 16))
 (segment (start 172.88038 68.40512) (end 177.466359 63.819141) (width 0.1524) (layer F.Cu) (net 16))
 (segment (start 180.566959 63.819141) (end 181.75986 62.62624) (width 0.1524) (layer F.Cu) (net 16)))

